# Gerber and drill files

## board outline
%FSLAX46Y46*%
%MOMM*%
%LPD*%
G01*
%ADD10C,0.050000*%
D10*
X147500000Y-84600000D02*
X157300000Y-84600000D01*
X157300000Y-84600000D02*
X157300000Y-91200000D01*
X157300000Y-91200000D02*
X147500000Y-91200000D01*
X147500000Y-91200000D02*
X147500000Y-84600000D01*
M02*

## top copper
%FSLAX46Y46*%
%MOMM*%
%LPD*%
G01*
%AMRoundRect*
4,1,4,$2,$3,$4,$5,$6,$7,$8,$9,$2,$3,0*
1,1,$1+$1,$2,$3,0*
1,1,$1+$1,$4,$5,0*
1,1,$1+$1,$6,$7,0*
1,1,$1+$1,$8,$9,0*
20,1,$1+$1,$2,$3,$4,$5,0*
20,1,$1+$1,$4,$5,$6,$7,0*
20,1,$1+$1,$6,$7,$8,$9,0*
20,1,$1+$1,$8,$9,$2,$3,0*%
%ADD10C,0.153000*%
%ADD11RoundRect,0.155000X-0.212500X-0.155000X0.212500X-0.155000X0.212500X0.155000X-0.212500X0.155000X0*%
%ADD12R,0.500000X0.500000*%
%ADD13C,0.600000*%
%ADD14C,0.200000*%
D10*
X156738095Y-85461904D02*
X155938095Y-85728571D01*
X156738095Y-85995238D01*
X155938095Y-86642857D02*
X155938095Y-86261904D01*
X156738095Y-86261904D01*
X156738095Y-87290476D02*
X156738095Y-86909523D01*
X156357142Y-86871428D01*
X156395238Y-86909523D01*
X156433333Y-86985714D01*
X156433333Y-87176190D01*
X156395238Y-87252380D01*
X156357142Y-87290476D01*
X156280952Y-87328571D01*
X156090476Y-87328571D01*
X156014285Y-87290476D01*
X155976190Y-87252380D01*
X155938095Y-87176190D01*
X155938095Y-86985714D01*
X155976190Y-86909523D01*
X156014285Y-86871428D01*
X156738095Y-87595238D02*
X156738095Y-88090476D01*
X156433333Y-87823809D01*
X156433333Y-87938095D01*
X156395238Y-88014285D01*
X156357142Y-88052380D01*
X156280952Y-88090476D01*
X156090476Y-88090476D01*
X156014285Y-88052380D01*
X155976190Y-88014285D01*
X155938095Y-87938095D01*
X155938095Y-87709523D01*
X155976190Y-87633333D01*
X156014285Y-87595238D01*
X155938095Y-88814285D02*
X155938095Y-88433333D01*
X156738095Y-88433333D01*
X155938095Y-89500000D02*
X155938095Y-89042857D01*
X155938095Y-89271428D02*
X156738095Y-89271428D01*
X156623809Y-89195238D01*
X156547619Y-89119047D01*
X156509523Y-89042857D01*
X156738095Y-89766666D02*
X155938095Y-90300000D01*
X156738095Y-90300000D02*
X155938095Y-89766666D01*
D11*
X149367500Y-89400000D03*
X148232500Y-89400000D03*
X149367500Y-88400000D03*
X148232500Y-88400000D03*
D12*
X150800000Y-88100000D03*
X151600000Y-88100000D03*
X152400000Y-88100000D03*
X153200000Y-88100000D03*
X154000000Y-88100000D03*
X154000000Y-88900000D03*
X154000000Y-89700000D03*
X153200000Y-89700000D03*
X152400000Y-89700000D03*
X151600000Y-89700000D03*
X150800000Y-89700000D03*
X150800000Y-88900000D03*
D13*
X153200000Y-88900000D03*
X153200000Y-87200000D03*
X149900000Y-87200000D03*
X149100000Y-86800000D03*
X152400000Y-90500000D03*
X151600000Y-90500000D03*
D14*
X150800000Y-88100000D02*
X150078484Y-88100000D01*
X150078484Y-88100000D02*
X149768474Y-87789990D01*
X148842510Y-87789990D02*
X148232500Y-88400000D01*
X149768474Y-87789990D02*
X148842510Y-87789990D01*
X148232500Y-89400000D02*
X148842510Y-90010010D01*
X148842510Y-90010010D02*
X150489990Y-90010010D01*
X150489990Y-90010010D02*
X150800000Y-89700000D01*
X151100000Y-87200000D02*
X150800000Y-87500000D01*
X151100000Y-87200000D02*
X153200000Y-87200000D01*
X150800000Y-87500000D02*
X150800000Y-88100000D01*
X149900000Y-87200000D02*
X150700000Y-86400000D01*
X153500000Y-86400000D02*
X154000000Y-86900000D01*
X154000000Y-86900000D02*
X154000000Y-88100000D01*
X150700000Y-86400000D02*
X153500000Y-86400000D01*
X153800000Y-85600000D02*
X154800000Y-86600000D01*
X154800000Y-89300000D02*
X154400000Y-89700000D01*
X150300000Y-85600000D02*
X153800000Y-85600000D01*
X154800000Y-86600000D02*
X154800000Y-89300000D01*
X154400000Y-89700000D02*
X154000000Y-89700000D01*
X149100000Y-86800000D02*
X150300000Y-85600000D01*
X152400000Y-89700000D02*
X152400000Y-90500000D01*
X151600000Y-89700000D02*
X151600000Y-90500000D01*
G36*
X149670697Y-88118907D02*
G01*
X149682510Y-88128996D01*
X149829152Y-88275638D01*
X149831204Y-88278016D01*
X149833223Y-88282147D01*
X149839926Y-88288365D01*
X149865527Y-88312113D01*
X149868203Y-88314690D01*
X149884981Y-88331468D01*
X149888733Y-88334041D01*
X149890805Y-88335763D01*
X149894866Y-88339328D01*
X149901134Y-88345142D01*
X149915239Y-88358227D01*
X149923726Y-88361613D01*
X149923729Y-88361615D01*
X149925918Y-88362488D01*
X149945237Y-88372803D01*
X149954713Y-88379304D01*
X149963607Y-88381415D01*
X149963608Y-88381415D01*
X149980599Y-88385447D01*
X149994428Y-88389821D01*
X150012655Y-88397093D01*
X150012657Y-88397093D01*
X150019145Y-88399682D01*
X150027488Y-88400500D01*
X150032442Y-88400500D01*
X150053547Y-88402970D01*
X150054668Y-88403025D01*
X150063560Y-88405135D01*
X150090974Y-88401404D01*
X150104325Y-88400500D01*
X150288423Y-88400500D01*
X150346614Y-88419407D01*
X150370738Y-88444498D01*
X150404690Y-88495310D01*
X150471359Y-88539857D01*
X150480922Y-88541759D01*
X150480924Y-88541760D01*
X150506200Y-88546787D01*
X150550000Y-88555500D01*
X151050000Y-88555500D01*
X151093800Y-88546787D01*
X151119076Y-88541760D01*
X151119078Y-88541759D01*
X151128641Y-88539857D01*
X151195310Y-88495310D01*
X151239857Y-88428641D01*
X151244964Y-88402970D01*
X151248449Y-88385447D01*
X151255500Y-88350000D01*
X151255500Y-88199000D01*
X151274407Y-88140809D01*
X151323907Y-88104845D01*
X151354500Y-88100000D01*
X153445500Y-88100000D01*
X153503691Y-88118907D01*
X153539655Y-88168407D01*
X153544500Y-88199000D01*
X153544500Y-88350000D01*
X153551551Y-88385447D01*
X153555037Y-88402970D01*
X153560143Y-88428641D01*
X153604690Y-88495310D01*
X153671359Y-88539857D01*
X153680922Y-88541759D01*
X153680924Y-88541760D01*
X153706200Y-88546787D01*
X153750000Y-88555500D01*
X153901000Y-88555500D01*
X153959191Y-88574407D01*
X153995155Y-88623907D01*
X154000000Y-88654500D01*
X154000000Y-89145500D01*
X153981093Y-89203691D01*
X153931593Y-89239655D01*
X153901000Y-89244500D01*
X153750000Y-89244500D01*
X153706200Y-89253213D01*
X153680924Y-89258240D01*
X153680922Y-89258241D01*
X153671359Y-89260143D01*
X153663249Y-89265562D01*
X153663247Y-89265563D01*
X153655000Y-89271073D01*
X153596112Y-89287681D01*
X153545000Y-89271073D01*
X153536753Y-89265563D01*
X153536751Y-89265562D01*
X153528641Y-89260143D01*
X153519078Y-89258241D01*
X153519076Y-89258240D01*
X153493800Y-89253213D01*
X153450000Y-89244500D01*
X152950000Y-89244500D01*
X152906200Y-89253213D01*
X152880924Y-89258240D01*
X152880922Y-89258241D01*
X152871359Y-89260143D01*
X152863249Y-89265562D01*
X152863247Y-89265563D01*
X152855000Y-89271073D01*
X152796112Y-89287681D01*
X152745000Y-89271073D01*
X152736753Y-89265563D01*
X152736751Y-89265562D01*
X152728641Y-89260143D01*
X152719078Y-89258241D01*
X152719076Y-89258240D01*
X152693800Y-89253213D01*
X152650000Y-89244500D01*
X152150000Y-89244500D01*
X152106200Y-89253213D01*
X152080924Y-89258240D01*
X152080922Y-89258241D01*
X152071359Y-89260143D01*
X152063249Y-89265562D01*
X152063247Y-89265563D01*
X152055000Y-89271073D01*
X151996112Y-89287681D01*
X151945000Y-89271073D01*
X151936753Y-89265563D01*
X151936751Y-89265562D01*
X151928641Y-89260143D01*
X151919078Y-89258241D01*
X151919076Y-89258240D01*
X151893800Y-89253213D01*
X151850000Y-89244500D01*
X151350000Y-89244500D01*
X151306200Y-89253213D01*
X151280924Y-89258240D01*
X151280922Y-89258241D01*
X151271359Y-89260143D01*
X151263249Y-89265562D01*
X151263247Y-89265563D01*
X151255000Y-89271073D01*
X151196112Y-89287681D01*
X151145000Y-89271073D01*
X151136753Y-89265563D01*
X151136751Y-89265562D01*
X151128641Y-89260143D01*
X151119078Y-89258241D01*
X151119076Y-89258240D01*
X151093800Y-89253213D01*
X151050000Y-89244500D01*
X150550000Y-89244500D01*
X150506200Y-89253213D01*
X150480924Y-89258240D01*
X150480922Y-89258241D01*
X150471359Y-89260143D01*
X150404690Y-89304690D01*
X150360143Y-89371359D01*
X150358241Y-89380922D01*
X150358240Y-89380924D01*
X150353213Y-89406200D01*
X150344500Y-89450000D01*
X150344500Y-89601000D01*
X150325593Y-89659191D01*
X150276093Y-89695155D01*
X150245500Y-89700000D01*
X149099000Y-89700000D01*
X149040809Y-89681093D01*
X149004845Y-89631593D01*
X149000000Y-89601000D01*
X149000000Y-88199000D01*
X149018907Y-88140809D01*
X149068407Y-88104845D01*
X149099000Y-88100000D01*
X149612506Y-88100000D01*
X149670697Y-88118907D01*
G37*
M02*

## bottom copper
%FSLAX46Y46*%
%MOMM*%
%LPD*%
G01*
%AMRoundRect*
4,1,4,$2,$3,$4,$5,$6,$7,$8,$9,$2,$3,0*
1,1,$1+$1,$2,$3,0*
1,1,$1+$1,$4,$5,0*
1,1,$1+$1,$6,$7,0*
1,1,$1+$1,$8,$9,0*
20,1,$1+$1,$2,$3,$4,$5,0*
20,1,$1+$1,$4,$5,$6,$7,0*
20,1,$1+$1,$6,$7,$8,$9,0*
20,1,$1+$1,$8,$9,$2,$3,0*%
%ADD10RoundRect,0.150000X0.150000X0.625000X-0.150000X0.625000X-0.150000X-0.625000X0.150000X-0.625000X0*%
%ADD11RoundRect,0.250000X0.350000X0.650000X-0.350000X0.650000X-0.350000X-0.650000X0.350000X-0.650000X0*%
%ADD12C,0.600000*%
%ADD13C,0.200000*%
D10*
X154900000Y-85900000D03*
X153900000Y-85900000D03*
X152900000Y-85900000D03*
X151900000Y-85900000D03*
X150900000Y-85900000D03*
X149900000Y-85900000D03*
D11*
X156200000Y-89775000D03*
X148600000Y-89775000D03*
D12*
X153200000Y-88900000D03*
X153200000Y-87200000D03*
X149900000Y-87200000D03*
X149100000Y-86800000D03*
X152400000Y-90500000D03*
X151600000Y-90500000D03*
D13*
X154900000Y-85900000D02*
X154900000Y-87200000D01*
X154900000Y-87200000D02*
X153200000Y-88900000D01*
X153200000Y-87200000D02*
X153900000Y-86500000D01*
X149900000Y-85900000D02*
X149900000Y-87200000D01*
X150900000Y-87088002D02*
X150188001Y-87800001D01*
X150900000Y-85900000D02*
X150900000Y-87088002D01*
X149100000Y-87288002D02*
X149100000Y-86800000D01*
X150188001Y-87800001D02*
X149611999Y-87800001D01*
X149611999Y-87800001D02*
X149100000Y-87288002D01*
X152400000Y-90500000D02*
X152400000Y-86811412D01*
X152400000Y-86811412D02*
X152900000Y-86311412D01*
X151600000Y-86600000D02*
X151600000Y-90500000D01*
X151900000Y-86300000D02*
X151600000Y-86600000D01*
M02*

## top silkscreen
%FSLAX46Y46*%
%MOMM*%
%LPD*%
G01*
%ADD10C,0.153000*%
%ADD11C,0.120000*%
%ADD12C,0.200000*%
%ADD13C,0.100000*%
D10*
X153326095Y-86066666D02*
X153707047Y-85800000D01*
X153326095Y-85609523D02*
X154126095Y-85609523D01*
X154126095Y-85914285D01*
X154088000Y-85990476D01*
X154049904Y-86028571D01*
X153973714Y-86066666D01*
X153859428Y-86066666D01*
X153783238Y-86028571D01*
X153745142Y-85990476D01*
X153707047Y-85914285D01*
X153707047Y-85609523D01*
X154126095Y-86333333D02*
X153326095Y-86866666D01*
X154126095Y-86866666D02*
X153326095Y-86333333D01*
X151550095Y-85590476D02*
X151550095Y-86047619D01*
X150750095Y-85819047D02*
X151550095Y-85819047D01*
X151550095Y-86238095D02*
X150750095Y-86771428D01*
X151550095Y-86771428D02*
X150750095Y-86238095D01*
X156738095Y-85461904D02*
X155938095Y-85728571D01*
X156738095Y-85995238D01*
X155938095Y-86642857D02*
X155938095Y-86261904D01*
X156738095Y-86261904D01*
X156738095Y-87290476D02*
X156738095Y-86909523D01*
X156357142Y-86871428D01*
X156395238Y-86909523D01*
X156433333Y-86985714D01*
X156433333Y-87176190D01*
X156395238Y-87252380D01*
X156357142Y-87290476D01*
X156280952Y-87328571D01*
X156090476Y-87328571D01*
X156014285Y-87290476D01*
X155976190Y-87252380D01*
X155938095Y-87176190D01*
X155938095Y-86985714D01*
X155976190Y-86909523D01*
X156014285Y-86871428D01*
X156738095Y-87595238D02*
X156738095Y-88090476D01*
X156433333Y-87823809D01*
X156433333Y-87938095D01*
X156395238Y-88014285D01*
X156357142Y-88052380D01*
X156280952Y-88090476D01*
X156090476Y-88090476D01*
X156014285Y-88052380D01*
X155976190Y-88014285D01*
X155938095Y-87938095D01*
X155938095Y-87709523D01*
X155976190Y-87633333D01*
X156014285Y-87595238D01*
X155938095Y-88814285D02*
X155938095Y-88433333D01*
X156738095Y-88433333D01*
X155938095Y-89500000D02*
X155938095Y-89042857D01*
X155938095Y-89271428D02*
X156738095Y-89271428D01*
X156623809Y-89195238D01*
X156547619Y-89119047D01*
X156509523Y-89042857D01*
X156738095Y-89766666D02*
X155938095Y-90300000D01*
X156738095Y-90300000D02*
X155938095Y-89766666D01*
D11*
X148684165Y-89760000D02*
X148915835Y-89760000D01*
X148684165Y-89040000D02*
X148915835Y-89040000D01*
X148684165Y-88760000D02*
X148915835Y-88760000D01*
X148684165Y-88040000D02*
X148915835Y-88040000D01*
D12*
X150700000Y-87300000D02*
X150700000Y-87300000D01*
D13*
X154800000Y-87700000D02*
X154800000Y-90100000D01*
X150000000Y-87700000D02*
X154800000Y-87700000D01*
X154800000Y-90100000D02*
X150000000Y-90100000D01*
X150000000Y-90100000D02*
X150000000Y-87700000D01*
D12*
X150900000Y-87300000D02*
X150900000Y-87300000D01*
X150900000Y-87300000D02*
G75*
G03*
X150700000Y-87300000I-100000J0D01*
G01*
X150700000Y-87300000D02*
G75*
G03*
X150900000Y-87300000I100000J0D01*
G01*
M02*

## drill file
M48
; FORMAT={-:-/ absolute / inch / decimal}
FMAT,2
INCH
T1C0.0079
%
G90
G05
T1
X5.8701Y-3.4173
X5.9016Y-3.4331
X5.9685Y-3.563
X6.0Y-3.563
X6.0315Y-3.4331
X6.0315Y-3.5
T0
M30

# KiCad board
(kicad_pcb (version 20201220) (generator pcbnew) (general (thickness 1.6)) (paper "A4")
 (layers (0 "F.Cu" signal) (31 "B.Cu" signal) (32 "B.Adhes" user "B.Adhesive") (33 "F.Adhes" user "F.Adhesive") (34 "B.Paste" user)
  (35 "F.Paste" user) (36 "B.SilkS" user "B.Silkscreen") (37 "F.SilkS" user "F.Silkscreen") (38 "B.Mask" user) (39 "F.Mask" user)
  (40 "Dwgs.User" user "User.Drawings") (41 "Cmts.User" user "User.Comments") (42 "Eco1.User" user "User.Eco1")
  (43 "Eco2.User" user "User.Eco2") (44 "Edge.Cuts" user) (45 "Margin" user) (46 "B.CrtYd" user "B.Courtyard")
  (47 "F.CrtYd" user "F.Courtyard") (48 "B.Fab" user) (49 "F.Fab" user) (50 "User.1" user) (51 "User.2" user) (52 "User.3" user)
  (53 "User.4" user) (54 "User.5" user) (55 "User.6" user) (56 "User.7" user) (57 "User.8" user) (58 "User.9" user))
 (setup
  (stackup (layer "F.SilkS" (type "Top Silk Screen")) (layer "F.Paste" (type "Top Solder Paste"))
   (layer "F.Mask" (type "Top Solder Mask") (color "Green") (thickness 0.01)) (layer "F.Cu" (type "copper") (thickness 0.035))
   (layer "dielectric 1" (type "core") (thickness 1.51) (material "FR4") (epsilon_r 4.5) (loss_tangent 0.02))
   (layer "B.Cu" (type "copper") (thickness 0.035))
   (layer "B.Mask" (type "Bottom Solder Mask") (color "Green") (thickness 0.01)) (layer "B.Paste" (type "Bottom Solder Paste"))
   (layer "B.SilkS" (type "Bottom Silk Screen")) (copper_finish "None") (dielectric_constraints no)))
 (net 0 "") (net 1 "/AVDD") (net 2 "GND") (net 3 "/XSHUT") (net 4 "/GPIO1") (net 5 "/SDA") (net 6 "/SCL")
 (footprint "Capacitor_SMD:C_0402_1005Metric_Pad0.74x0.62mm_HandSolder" (layer "F.Cu") (at 148.8 89.4)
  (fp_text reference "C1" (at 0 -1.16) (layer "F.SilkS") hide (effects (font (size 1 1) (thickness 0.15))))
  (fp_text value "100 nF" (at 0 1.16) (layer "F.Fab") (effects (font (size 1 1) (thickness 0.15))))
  (fp_line (start -0.115835 -0.36) (end 0.115835 -0.36) (layer "F.SilkS") (width 0.12))
  (fp_line (start -0.115835 0.36) (end 0.115835 0.36) (layer "F.SilkS") (width 0.12))
  (pad "1" smd roundrect (at -0.5675 0) (size 0.735 0.62) (layers "F.Cu" "F.Paste" "F.Mask") (roundrect_rratio 0.25) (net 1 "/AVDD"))
  (pad "2" smd roundrect (at 0.5675 0) (size 0.735 0.62) (layers "F.Cu" "F.Paste" "F.Mask") (roundrect_rratio 0.25) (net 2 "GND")))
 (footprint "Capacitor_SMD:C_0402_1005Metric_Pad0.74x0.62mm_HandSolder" (layer "F.Cu") (at 148.8 88.4)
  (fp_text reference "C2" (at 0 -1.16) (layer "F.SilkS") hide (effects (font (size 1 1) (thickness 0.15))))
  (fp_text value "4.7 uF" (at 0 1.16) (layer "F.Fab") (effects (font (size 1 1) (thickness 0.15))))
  (fp_line (start -0.115835 0.36) (end 0.115835 0.36) (layer "F.SilkS") (width 0.12))
  (fp_line (start -0.115835 -0.36) (end 0.115835 -0.36) (layer "F.SilkS") (width 0.12))
  (pad "1" smd roundrect (at -0.5675 0) (size 0.735 0.62) (layers "F.Cu" "F.Paste" "F.Mask") (roundrect_rratio 0.25) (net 1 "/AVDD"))
  (pad "2" smd roundrect (at 0.5675 0) (size 0.735 0.62) (layers "F.Cu" "F.Paste" "F.Mask") (roundrect_rratio 0.25) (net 2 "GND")))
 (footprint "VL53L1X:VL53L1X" (layer "F.Cu") (at 152.4 88.9)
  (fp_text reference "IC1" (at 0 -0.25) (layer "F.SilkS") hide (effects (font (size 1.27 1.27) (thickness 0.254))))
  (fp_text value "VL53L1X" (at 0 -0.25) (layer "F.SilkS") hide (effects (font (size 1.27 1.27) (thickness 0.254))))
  (fp_line (start -1.7 -1.6) (end -1.7 -1.6) (layer "F.SilkS") (width 0.2))
  (fp_line (start 2.4 -1.2) (end 2.4 1.2) (layer "F.SilkS") (width 0.1))
  (fp_line (start -2.4 -1.2) (end 2.4 -1.2) (layer "F.SilkS") (width 0.1))
  (fp_line (start 2.4 1.2) (end -2.4 1.2) (layer "F.SilkS") (width 0.1))
  (fp_line (start -2.4 1.2) (end -2.4 -1.2) (layer "F.SilkS") (width 0.1))
  (fp_line (start -1.5 -1.6) (end -1.5 -1.6) (layer "F.SilkS") (width 0.2))
  (fp_arc (start -1.6 -1.6) (end -1.7 -1.6) (angle 180) (layer "F.SilkS") (width 0.2))
  (fp_arc (start -1.6 -1.6) (end -1.5 -1.6) (angle 180) (layer "F.SilkS") (width 0.2))
  (pad "1" smd rect (at -1.6 -0.8 90) (size 0.5 0.5) (layers "F.Cu" "F.Paste" "F.Mask") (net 1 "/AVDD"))
  (pad "2" smd rect (at -0.8 -0.8 90) (size 0.5 0.5) (layers "F.Cu" "F.Paste" "F.Mask") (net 2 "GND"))
  (pad "3" smd rect (at 0 -0.8 90) (size 0.5 0.5) (layers "F.Cu" "F.Paste" "F.Mask") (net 2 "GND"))
  (pad "4" smd rect (at 0.8 -0.8 90) (size 0.5 0.5) (layers "F.Cu" "F.Paste" "F.Mask") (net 2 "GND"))
  (pad "5" smd rect (at 1.6 -0.8 90) (size 0.5 0.5) (layers "F.Cu" "F.Paste" "F.Mask") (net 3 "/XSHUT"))
  (pad "6" smd rect (at 1.6 0 90) (size 0.5 0.5) (layers "F.Cu" "F.Paste" "F.Mask") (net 2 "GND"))
  (pad "7" smd rect (at 1.6 0.8 90) (size 0.5 0.5) (layers "F.Cu" "F.Paste" "F.Mask") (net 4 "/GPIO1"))
  (pad "8" smd rect (at 0.8 0.8 90) (size 0.5 0.5) (layers "F.Cu" "F.Paste" "F.Mask"))
  (pad "9" smd rect (at 0 0.8 90) (size 0.5 0.5) (layers "F.Cu" "F.Paste" "F.Mask") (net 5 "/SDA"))
  (pad "10" smd rect (at -0.8 0.8 90) (size 0.5 0.5) (layers "F.Cu" "F.Paste" "F.Mask") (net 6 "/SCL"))
  (pad "11" smd rect (at -1.6 0.8 90) (size 0.5 0.5) (layers "F.Cu" "F.Paste" "F.Mask") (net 1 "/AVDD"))
  (pad "12" smd rect (at -1.6 0 90) (size 0.5 0.5) (layers "F.Cu" "F.Paste" "F.Mask") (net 2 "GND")))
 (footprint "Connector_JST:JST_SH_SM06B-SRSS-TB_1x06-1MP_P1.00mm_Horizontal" (layer "B.Cu") (at 152.4 87.9 180)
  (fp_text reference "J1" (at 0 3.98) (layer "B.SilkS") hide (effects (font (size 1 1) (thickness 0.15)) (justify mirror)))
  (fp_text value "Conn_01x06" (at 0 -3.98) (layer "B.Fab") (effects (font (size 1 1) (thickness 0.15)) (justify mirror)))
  (pad "1" smd roundrect (at -2.5 2 180) (size 0.6 1.55) (layers "B.Cu" "B.Paste" "B.Mask") (roundrect_rratio 0.25) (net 2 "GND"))
  (pad "2" smd roundrect (at -1.5 2 180) (size 0.6 1.55) (layers "B.Cu" "B.Paste" "B.Mask") (roundrect_rratio 0.25) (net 1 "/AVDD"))
  (pad "3" smd roundrect (at -0.5 2 180) (size 0.6 1.55) (layers "B.Cu" "B.Paste" "B.Mask") (roundrect_rratio 0.25) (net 5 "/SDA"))
  (pad "4" smd roundrect (at 0.5 2 180) (size 0.6 1.55) (layers "B.Cu" "B.Paste" "B.Mask") (roundrect_rratio 0.25) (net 6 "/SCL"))
  (pad "5" smd roundrect (at 1.5 2 180) (size 0.6 1.55) (layers "B.Cu" "B.Paste" "B.Mask") (roundrect_rratio 0.25) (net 4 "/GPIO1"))
  (pad "6" smd roundrect (at 2.5 2 180) (size 0.6 1.55) (layers "B.Cu" "B.Paste" "B.Mask") (roundrect_rratio 0.25) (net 3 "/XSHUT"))
  (pad "MP" smd roundrect (at -3.8 -1.875 180) (size 1.2 1.8) (layers "B.Cu" "B.Paste" "B.Mask") (roundrect_rratio 0.2083333333333333))
  (pad "MP" smd roundrect (at 3.8 -1.875 180) (size 1.2 1.8) (layers "B.Cu" "B.Paste" "B.Mask") (roundrect_rratio 0.2083333333333333)))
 (gr_rect (start 147.5 84.6) (end 157.3 91.2) (layer "Edge.Cuts") (width 0.05) (fill none))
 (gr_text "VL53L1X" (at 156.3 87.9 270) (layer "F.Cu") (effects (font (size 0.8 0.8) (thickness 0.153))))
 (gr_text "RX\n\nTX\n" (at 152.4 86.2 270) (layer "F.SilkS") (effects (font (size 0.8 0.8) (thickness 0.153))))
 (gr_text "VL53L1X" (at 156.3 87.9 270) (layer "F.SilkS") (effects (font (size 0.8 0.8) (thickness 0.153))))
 (via (at 153.2 88.9) (size 0.6) (drill 0.2) (layers "F.Cu" "B.Cu") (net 2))
 (segment (start 154.9 85.9) (end 154.9 87.2) (width 0.2) (layer "B.Cu") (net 2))
 (segment (start 154.9 87.2) (end 153.2 88.9) (width 0.2) (layer "B.Cu") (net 2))
 (segment (start 148.84251 90.01001) (end 150.48999 90.01001) (width 0.2) (layer "F.Cu") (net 1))
 (segment (start 150.078484 88.1) (end 149.768474 87.78999) (width 0.2) (layer "F.Cu") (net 1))
 (segment (start 150.48999 90.01001) (end 150.8 89.7) (width 0.2) (layer "F.Cu") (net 1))
 (segment (start 151.1 87.2) (end 150.8 87.5) (width 0.2) (layer "F.Cu") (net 1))
 (segment (start 148.84251 87.78999) (end 148.2325 88.4) (width 0.2) (layer "F.Cu") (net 1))
 (segment (start 150.8 88.1) (end 150.078484 88.1) (width 0.2) (layer "F.Cu") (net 1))
 (segment (start 149.768474 87.78999) (end 148.84251 87.78999) (width 0.2) (layer "F.Cu") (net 1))
 (segment (start 151.1 87.2) (end 153.2 87.2) (width 0.2) (layer "F.Cu") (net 1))
 (segment (start 150.8 87.5) (end 150.8 88.1) (width 0.2) (layer "F.Cu") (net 1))
 (segment (start 148.2325 89.4) (end 148.84251 90.01001) (width 0.2) (layer "F.Cu") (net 1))
 (via (at 153.2 87.2) (size 0.6) (drill 0.2) (layers "F.Cu" "B.Cu") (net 1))
 (segment (start 153.2 87.2) (end 153.9 86.5) (width 0.2) (layer "B.Cu") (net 1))
 (segment (start 149.9 87.2) (end 150.7 86.4) (width 0.2) (layer "F.Cu") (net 3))
 (segment (start 153.5 86.4) (end 154 86.9) (width 0.2) (layer "F.Cu") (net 3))
 (segment (start 154 86.9) (end 154 88.1) (width 0.2) (layer "F.Cu") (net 3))
 (segment (start 150.7 86.4) (end 153.5 86.4) (width 0.2) (layer "F.Cu") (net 3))
 (via (at 149.9 87.2) (size 0.6) (drill 0.2) (layers "F.Cu" "B.Cu") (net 3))
 (segment (start 149.9 85.9) (end 149.9 87.2) (width 0.2) (layer "B.Cu") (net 3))
 (segment (start 153.8 85.6) (end 154.8 86.6) (width 0.2) (layer "F.Cu") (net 4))
 (segment (start 154.8 89.3) (end 154.4 89.7) (width 0.2) (layer "F.Cu") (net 4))
 (segment (start 150.3 85.6) (end 153.8 85.6) (width 0.2) (layer "F.Cu") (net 4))
 (segment (start 154.8 86.6) (end 154.8 89.3) (width 0.2) (layer "F.Cu") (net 4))
 (segment (start 154.4 89.7) (end 154 89.7) (width 0.2) (layer "F.Cu") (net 4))
 (segment (start 149.1 86.8) (end 150.3 85.6) (width 0.2) (layer "F.Cu") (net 4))
 (via (at 149.1 86.8) (size 0.6) (drill 0.2) (layers "F.Cu" "B.Cu") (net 4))
 (segment (start 150.9 87.088002) (end 150.188001 87.800001) (width 0.2) (layer "B.Cu") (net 4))
 (segment (start 150.9 85.9) (end 150.9 87.088002) (width 0.2) (layer "B.Cu") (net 4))
 (segment (start 149.1 87.288002) (end 149.1 86.8) (width 0.2) (layer "B.Cu") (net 4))
 (segment (start 150.188001 87.800001) (end 149.611999 87.800001) (width 0.2) (layer "B.Cu") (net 4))
 (segment (start 149.611999 87.800001) (end 149.1 87.288002) (width 0.2) (layer "B.Cu") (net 4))
 (segment (start 152.4 89.7) (end 152.4 90.5) (width 0.2) (layer "F.Cu") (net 5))
 (via (at 152.4 90.5) (size 0.6) (drill 0.2) (layers "F.Cu" "B.Cu") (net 5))
 (segment (start 152.4 90.5) (end 152.4 86.811412) (width 0.2) (layer "B.Cu") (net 5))
 (segment (start 152.4 86.811412) (end 152.9 86.311412) (width 0.2) (layer "B.Cu") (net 5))
 (segment (start 151.6 89.7) (end 151.6 90.5) (width 0.2) (layer "F.Cu") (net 6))
 (via (at 151.6 90.5) (size 0.6) (drill 0.2) (layers "F.Cu" "B.Cu") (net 6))
 (segment (start 151.6 86.6) (end 151.6 90.5) (width 0.2) (layer "B.Cu") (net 6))
 (segment (start 151.9 86.3) (end 151.6 86.6) (width 0.2) (layer "B.Cu") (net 6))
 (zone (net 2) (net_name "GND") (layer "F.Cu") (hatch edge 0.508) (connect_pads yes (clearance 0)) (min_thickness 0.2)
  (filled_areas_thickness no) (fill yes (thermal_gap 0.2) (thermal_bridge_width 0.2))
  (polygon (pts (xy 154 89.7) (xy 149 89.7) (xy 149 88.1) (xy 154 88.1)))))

